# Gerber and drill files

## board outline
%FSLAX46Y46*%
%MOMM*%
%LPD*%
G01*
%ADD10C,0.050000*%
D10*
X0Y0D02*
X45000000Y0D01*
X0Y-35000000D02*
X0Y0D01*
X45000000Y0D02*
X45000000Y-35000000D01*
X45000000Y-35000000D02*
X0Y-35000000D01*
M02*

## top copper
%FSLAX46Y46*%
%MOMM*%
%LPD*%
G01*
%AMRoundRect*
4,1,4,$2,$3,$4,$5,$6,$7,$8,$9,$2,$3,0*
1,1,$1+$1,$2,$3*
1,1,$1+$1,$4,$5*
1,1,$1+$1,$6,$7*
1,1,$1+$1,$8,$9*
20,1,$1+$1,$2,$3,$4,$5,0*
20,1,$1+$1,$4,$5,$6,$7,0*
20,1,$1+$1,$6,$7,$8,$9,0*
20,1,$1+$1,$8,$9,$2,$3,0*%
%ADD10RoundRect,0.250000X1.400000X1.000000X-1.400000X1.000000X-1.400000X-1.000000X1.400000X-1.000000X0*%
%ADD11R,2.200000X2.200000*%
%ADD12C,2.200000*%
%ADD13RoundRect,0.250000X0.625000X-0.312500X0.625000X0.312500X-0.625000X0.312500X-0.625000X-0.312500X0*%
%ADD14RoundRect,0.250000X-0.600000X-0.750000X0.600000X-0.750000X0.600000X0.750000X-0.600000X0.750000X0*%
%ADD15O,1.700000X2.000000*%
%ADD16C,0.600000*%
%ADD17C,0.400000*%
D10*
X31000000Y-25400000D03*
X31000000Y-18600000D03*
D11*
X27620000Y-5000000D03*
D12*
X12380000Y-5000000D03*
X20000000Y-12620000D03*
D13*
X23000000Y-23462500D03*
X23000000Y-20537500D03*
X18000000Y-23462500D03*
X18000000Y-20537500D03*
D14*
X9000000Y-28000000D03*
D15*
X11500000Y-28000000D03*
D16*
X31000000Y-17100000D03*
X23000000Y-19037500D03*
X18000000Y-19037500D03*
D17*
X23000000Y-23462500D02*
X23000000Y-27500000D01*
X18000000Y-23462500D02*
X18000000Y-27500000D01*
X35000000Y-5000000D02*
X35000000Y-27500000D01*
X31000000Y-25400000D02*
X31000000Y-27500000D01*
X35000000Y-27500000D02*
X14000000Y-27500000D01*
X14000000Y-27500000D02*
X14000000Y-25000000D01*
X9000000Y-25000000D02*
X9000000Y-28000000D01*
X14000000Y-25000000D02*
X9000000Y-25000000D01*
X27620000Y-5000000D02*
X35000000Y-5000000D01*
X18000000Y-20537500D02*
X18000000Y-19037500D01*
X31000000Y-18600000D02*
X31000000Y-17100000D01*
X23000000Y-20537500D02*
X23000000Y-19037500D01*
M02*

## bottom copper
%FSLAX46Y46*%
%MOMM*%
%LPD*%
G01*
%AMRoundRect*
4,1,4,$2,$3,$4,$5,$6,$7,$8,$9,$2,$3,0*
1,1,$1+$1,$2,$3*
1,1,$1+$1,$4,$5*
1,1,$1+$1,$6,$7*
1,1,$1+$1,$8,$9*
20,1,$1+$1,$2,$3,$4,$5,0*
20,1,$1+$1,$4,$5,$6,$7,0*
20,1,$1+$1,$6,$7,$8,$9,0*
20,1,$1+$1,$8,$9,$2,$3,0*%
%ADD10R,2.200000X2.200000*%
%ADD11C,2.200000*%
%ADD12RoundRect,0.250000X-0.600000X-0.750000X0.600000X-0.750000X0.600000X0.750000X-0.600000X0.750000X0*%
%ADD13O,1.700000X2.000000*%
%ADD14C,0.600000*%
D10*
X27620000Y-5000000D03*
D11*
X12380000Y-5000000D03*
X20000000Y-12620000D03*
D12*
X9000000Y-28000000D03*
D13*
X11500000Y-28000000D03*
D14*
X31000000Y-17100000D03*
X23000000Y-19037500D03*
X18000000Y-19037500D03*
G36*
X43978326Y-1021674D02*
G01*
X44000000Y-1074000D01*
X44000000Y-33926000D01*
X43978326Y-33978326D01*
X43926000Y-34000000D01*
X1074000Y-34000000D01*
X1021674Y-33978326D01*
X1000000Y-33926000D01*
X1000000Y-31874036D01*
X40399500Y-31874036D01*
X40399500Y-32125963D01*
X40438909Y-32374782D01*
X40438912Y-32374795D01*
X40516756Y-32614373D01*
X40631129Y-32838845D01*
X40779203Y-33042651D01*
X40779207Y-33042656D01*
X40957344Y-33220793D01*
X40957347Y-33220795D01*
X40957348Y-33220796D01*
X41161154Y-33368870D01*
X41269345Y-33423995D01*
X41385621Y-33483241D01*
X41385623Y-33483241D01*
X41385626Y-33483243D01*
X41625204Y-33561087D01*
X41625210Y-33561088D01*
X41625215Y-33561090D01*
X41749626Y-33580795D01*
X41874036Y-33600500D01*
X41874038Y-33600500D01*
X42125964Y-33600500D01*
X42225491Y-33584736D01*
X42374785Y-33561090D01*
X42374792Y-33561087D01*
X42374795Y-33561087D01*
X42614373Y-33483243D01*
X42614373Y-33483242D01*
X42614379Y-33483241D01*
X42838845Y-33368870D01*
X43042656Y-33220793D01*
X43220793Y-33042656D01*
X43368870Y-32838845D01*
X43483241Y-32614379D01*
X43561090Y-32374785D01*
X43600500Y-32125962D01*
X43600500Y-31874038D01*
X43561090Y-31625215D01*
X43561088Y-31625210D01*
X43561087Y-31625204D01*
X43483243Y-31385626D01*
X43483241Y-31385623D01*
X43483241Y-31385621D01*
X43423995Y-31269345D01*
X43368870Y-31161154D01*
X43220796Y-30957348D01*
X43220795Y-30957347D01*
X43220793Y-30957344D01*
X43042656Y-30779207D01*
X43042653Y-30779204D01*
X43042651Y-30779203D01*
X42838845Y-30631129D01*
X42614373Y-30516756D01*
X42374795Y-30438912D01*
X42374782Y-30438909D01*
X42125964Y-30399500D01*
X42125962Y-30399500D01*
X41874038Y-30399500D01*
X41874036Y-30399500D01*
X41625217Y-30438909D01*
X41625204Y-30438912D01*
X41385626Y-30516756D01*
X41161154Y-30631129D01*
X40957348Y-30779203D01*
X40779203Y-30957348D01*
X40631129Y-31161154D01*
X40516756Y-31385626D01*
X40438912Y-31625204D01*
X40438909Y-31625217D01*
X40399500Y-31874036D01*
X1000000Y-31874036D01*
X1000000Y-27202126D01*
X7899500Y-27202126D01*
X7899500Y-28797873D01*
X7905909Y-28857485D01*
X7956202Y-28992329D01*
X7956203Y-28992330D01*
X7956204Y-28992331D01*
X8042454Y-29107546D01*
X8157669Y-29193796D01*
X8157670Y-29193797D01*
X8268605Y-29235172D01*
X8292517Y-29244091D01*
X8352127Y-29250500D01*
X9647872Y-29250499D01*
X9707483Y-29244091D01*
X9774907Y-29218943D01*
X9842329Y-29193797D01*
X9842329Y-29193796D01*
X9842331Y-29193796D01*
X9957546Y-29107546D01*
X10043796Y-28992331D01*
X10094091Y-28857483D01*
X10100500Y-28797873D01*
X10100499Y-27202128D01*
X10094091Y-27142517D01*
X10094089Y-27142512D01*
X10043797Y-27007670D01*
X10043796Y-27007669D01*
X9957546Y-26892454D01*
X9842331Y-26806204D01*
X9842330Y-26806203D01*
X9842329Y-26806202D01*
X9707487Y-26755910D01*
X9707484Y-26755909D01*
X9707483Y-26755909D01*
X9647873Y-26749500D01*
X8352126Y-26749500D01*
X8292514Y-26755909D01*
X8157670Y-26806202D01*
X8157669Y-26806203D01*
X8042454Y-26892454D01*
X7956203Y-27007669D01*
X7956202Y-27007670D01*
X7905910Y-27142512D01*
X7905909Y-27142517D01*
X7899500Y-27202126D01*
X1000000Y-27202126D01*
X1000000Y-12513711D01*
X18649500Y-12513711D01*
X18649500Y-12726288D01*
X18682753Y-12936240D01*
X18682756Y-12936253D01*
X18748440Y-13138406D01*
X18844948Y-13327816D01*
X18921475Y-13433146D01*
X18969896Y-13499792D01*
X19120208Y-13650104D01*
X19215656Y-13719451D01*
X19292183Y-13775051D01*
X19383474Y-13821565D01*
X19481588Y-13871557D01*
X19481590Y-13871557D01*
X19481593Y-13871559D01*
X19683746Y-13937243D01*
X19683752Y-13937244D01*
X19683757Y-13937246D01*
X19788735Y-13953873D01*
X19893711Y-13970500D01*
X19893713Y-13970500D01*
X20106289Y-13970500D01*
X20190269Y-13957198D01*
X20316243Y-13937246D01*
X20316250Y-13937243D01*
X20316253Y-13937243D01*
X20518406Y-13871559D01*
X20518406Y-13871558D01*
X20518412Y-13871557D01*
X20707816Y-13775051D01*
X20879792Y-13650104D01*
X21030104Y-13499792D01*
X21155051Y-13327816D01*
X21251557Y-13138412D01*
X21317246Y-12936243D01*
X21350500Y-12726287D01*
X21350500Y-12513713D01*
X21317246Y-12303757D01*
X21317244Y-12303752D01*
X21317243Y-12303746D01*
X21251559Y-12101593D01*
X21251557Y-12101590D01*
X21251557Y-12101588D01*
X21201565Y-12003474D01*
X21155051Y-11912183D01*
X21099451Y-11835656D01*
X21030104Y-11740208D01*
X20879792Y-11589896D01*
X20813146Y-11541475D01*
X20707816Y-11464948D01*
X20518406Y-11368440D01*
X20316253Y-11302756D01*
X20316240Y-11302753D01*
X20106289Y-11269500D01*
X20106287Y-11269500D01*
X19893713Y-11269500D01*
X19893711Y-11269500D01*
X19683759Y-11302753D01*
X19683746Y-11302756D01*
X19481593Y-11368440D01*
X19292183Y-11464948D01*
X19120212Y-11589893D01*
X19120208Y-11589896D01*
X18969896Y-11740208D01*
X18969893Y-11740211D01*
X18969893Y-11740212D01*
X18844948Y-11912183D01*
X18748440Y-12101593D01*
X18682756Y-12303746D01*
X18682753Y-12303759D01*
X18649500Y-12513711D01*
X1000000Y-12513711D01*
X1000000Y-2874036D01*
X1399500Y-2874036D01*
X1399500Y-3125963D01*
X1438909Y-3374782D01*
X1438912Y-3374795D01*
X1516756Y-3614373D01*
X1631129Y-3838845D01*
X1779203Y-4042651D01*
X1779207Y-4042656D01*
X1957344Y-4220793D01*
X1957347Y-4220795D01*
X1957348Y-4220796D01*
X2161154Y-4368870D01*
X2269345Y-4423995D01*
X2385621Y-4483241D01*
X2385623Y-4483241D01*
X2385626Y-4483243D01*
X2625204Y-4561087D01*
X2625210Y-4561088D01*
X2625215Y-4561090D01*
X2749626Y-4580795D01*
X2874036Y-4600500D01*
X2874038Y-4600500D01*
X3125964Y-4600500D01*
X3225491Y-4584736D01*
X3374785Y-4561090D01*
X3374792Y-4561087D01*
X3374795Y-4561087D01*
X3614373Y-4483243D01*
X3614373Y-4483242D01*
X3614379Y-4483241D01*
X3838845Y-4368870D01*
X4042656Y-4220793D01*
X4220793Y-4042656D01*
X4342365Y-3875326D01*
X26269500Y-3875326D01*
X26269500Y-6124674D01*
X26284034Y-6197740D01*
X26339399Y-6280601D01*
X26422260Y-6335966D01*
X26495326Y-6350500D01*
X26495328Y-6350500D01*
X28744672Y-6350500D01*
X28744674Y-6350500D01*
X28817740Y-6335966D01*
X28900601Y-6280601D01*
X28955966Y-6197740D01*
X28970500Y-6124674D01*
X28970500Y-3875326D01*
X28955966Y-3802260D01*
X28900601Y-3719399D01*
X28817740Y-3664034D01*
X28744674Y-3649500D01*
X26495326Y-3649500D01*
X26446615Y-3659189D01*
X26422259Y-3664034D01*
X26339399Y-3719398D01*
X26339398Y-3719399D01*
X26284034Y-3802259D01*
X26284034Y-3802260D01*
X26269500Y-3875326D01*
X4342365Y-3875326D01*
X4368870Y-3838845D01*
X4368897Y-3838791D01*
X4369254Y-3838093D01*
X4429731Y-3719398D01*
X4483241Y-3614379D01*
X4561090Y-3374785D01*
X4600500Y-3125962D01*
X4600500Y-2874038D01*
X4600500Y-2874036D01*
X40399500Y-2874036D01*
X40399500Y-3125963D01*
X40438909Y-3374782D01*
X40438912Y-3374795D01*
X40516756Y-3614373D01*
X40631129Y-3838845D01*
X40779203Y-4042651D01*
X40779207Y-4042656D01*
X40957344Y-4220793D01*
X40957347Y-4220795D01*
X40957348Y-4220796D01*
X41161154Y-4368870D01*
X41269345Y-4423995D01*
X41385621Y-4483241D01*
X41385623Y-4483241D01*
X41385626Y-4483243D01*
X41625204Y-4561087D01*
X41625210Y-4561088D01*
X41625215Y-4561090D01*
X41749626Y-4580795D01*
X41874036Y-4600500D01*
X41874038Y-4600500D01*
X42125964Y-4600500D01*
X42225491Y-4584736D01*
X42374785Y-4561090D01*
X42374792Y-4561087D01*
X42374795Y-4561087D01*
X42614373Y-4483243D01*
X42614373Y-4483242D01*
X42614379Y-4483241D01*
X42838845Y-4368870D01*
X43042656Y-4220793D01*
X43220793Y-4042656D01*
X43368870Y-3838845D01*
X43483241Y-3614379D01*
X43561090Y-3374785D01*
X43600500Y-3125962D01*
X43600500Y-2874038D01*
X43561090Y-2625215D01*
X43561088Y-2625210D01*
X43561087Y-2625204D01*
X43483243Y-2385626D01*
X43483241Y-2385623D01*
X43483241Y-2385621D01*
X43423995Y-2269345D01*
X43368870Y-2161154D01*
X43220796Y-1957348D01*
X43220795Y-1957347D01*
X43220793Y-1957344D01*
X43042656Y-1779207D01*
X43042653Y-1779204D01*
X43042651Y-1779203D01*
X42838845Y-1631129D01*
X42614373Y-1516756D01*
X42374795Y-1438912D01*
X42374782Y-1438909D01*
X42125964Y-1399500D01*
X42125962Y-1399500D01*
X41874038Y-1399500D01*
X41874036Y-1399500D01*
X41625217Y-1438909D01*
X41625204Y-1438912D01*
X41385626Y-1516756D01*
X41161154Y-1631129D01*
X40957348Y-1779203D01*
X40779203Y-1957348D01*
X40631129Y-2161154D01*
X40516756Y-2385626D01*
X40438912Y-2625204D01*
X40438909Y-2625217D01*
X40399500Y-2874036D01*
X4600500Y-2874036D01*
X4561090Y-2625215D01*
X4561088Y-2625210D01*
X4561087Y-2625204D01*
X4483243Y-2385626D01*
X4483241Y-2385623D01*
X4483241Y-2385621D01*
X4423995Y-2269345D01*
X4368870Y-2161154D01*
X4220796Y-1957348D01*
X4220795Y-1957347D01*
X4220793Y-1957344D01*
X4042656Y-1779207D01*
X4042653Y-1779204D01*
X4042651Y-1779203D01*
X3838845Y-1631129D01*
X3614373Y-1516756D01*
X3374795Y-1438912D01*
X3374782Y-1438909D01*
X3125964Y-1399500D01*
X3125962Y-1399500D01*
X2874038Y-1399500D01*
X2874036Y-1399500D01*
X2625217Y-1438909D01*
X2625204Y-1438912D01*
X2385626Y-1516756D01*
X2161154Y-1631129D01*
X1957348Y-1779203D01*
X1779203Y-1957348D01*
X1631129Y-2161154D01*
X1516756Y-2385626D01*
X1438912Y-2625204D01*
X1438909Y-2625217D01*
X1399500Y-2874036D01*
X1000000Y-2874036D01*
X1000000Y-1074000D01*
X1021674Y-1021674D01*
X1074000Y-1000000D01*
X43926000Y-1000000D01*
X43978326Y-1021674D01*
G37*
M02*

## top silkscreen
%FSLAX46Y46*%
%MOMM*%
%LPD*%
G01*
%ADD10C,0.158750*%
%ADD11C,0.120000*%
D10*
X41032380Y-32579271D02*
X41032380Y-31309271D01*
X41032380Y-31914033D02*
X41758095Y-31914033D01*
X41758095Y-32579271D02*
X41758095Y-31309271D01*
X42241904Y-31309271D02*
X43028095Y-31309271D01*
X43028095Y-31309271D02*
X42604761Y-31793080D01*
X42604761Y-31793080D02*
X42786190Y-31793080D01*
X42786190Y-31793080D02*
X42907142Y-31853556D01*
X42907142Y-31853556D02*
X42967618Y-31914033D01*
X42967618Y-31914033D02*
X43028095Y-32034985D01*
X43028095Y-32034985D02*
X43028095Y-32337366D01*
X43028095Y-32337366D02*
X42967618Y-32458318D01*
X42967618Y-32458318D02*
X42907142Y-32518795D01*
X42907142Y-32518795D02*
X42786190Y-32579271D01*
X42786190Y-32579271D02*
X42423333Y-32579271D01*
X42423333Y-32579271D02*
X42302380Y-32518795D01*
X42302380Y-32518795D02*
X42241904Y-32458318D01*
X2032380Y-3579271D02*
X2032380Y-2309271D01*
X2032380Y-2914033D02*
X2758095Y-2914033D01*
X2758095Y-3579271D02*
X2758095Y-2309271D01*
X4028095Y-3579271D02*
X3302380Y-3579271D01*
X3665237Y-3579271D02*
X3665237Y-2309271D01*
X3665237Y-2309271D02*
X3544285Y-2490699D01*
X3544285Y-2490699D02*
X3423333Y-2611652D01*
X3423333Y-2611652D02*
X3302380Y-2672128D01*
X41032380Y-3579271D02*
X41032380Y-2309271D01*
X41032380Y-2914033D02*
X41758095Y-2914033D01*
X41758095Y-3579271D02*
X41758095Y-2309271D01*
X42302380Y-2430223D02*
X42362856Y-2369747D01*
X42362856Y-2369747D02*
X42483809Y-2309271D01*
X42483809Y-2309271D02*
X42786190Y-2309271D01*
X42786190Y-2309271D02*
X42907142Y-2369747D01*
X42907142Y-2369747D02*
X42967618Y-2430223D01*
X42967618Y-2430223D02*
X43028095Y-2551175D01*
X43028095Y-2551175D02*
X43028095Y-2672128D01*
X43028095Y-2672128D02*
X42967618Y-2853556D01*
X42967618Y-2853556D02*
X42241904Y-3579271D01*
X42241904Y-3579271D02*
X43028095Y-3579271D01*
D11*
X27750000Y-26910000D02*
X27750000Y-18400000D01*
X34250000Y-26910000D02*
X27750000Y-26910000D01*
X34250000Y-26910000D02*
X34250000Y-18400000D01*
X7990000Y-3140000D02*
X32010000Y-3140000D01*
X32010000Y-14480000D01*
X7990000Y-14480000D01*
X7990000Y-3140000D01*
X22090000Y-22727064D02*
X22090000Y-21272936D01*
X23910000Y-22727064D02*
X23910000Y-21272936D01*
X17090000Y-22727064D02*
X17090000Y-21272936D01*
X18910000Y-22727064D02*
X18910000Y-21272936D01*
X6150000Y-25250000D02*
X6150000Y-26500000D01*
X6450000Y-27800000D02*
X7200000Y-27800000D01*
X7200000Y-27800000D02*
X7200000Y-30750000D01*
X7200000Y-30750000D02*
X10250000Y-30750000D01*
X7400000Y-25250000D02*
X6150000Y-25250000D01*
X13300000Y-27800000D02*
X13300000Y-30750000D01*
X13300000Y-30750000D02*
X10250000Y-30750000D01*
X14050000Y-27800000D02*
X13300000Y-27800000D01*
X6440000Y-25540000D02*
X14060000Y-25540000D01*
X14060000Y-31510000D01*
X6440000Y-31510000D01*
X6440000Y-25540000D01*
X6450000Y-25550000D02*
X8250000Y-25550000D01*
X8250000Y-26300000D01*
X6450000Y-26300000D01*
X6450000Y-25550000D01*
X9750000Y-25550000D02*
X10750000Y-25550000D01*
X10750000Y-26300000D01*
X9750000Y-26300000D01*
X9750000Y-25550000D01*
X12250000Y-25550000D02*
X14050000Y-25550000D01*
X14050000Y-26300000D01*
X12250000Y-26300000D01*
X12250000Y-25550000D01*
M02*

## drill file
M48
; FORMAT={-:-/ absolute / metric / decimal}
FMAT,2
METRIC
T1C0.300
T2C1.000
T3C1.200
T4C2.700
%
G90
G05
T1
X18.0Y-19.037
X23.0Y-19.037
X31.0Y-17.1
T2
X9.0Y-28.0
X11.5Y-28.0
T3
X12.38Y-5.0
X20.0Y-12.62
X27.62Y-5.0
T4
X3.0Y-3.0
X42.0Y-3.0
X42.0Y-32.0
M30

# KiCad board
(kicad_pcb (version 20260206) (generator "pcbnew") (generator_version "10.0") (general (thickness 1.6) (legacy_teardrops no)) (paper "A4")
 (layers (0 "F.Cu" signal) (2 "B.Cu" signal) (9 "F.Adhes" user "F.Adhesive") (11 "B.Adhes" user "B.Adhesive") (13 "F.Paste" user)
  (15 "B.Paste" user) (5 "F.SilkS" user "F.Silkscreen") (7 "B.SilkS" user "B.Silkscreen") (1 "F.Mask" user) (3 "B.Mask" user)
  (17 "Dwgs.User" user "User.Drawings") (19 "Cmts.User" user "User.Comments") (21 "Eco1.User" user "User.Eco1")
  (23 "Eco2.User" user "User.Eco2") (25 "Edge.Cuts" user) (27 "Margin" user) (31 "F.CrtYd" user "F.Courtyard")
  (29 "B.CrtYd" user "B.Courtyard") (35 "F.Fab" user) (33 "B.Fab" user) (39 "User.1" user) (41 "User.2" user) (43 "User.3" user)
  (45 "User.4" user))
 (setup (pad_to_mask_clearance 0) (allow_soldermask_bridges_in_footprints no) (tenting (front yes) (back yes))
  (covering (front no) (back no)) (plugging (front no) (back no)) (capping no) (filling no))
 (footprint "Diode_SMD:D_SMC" (layer "F.Cu") (at 31 22 90)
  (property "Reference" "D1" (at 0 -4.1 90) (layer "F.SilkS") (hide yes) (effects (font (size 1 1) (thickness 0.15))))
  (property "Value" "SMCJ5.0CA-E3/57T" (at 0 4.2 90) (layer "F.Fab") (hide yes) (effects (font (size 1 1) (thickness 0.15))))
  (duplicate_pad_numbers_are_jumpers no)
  (fp_line (start -4.91 -3.25) (end 3.6 -3.25) (stroke (width 0.12) (type solid)) (layer "F.SilkS"))
  (fp_line (start -4.91 3.25) (end -4.91 -3.25) (stroke (width 0.12) (type solid)) (layer "F.SilkS"))
  (fp_line (start -4.91 3.25) (end 3.6 3.25) (stroke (width 0.12) (type solid)) (layer "F.SilkS"))
  (pad "1" smd roundrect (at -3.4 0 180) (size 3.3 2.5) (layers "F.Cu" "F.Mask" "F.Paste") (roundrect_rratio 0.1) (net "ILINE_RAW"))
  (pad "2" smd roundrect (at 3.4 0 180) (size 3.3 2.5) (layers "F.Cu" "F.Mask" "F.Paste") (roundrect_rratio 0.1) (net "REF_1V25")))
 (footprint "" (layer "F.Cu") (at 42 32)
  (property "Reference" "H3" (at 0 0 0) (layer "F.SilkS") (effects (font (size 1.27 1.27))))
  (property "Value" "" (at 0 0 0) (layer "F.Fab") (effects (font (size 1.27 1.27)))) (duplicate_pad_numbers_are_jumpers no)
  (pad "" np_thru_hole circle (at 0 0) (size 2.7 2.7) (drill 2.7) (layers "*.Cu")))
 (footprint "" (layer "F.Cu") (at 3 3)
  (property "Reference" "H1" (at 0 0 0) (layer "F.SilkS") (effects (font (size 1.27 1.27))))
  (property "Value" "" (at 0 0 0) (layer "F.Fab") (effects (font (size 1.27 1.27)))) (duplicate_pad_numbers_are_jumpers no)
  (pad "" np_thru_hole circle (at 0 0) (size 2.7 2.7) (drill 2.7) (layers "*.Cu")))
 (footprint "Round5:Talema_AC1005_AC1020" (layer "F.Cu") (at 20 5)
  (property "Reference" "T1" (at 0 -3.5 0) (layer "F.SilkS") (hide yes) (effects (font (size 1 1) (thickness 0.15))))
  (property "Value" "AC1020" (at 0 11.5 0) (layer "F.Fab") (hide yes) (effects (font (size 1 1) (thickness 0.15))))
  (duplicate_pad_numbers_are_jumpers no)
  (fp_rect (start -12.01 -1.86) (end 12.01 9.48) (stroke (width 0.12) (type default)) (fill no) (layer "F.SilkS"))
  (pad "1" thru_hole rect (at 7.62 0) (size 2.2 2.2) (drill 1.2) (layers "*.Cu" "*.Mask") (remove_unused_layers no) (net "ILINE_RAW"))
  (pad "2" thru_hole circle (at -7.62 0) (size 2.2 2.2) (drill 1.2) (layers "*.Cu" "*.Mask") (remove_unused_layers no) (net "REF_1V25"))
  (pad "3" thru_hole circle (at 0 7.62) (size 2.2 2.2) (drill 1.2) (layers "*.Cu" "*.Mask") (remove_unused_layers no)
   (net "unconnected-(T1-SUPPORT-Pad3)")))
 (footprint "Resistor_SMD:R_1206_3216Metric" (layer "F.Cu") (at 23 22 90)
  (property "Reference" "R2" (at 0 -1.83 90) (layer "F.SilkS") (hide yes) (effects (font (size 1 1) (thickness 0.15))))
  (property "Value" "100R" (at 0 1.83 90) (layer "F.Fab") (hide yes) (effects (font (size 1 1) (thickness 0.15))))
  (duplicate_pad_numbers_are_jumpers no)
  (fp_line (start -0.727064 -0.91) (end 0.727064 -0.91) (stroke (width 0.12) (type solid)) (layer "F.SilkS"))
  (fp_line (start -0.727064 0.91) (end 0.727064 0.91) (stroke (width 0.12) (type solid)) (layer "F.SilkS"))
  (pad "1" smd roundrect (at -1.4625 0 90) (size 1.125 1.75) (layers "F.Cu" "F.Mask" "F.Paste") (roundrect_rratio 0.222222)
   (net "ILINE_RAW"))
  (pad "2" smd roundrect (at 1.4625 0 90) (size 1.125 1.75) (layers "F.Cu" "F.Mask" "F.Paste") (roundrect_rratio 0.222222) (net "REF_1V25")))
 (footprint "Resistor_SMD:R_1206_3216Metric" (layer "F.Cu") (at 18 22 90)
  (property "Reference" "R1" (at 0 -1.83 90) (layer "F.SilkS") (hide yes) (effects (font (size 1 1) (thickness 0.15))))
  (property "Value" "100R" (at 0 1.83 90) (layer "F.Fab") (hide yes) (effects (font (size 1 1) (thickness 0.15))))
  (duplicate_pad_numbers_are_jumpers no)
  (fp_line (start -0.727064 -0.91) (end 0.727064 -0.91) (stroke (width 0.12) (type solid)) (layer "F.SilkS"))
  (fp_line (start -0.727064 0.91) (end 0.727064 0.91) (stroke (width 0.12) (type solid)) (layer "F.SilkS"))
  (pad "1" smd roundrect (at -1.4625 0 90) (size 1.125 1.75) (layers "F.Cu" "F.Mask" "F.Paste") (roundrect_rratio 0.222222)
   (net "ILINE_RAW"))
  (pad "2" smd roundrect (at 1.4625 0 90) (size 1.125 1.75) (layers "F.Cu" "F.Mask" "F.Paste") (roundrect_rratio 0.222222) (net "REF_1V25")))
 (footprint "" (layer "F.Cu") (at 42 3)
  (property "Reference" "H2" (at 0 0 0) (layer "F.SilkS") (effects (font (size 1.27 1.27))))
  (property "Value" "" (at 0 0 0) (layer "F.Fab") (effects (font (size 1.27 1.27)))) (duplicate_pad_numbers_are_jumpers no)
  (pad "" np_thru_hole circle (at 0 0) (size 2.7 2.7) (drill 2.7) (layers "*.Cu")))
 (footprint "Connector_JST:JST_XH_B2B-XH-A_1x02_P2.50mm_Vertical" (layer "F.Cu") (at 9 28)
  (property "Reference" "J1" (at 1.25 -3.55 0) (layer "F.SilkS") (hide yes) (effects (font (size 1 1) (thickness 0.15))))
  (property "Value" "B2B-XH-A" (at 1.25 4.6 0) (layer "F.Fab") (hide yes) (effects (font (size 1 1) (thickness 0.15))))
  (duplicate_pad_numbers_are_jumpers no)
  (fp_line (start -2.85 -2.75) (end -2.85 -1.5) (stroke (width 0.12) (type solid)) (layer "F.SilkS"))
  (fp_line (start -2.55 -0.2) (end -1.8 -0.2) (stroke (width 0.12) (type solid)) (layer "F.SilkS"))
  (fp_line (start -1.8 -0.2) (end -1.8 2.75) (stroke (width 0.12) (type solid)) (layer "F.SilkS"))
  (fp_line (start -1.8 2.75) (end 1.25 2.75) (stroke (width 0.12) (type solid)) (layer "F.SilkS"))
  (fp_line (start -1.6 -2.75) (end -2.85 -2.75) (stroke (width 0.12) (type solid)) (layer "F.SilkS"))
  (fp_line (start 4.3 -0.2) (end 4.3 2.75) (stroke (width 0.12) (type solid)) (layer "F.SilkS"))
  (fp_line (start 4.3 2.75) (end 1.25 2.75) (stroke (width 0.12) (type solid)) (layer "F.SilkS"))
  (fp_line (start 5.05 -0.2) (end 4.3 -0.2) (stroke (width 0.12) (type solid)) (layer "F.SilkS"))
  (fp_rect (start -2.56 -2.46) (end 5.06 3.51) (stroke (width 0.12) (type solid)) (fill no) (layer "F.SilkS"))
  (fp_rect (start -2.55 -2.45) (end -0.75 -1.7) (stroke (width 0.12) (type solid)) (fill no) (layer "F.SilkS"))
  (fp_rect (start 0.75 -2.45) (end 1.75 -1.7) (stroke (width 0.12) (type solid)) (fill no) (layer "F.SilkS"))
  (fp_rect (start 3.25 -2.45) (end 5.05 -1.7) (stroke (width 0.12) (type solid)) (fill no) (layer "F.SilkS"))
  (pad "1" thru_hole roundrect (at 0 0) (size 1.7 2) (drill 1) (layers "*.Cu" "*.Mask") (remove_unused_layers no)
   (roundrect_rratio 0.147059) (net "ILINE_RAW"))
  (pad "2" thru_hole oval (at 2.5 0) (size 1.7 2) (drill 1) (layers "*.Cu" "*.Mask") (remove_unused_layers no) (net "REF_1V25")))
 (gr_line (start 0 0) (end 45 0) (stroke (width 0.05) (type default)) (layer "Edge.Cuts"))
 (gr_line (start 0 35) (end 0 0) (stroke (width 0.05) (type default)) (layer "Edge.Cuts"))
 (gr_line (start 45 0) (end 45 35) (stroke (width 0.05) (type default)) (layer "Edge.Cuts"))
 (gr_line (start 45 35) (end 0 35) (stroke (width 0.05) (type default)) (layer "Edge.Cuts"))
 (segment (start 23 23.4625) (end 23 27.5) (width 0.4) (layer "F.Cu") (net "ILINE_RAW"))
 (segment (start 18 23.4625) (end 18 27.5) (width 0.4) (layer "F.Cu") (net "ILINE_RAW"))
 (segment (start 35 5) (end 35 27.5) (width 0.4) (layer "F.Cu") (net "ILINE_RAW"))
 (segment (start 31 25.4) (end 31 27.5) (width 0.4) (layer "F.Cu") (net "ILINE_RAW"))
 (segment (start 35 27.5) (end 14 27.5) (width 0.4) (layer "F.Cu") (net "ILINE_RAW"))
 (segment (start 14 27.5) (end 14 25) (width 0.4) (layer "F.Cu") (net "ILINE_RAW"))
 (segment (start 9 25) (end 9 28) (width 0.4) (layer "F.Cu") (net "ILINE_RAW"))
 (segment (start 14 25) (end 9 25) (width 0.4) (layer "F.Cu") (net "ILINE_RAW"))
 (segment (start 27.62 5) (end 35 5) (width 0.4) (layer "F.Cu") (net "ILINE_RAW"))
 (segment (start 18 20.5375) (end 18 19.0375) (width 0.4) (layer "F.Cu") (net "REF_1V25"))
 (segment (start 31 18.6) (end 31 17.1) (width 0.4) (layer "F.Cu") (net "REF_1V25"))
 (segment (start 23 20.5375) (end 23 19.0375) (width 0.4) (layer "F.Cu") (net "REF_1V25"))
 (via (at 31 17.1) (size 0.6) (drill 0.3) (layers "F.Cu" "B.Cu") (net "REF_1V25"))
 (via (at 23 19.0375) (size 0.6) (drill 0.3) (layers "F.Cu" "B.Cu") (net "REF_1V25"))
 (via (at 18 19.0375) (size 0.6) (drill 0.3) (layers "F.Cu" "B.Cu") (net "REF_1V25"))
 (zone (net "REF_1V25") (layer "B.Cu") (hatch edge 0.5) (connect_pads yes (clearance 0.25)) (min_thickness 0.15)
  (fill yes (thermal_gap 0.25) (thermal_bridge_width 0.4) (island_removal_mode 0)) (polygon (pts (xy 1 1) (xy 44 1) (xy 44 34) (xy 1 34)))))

